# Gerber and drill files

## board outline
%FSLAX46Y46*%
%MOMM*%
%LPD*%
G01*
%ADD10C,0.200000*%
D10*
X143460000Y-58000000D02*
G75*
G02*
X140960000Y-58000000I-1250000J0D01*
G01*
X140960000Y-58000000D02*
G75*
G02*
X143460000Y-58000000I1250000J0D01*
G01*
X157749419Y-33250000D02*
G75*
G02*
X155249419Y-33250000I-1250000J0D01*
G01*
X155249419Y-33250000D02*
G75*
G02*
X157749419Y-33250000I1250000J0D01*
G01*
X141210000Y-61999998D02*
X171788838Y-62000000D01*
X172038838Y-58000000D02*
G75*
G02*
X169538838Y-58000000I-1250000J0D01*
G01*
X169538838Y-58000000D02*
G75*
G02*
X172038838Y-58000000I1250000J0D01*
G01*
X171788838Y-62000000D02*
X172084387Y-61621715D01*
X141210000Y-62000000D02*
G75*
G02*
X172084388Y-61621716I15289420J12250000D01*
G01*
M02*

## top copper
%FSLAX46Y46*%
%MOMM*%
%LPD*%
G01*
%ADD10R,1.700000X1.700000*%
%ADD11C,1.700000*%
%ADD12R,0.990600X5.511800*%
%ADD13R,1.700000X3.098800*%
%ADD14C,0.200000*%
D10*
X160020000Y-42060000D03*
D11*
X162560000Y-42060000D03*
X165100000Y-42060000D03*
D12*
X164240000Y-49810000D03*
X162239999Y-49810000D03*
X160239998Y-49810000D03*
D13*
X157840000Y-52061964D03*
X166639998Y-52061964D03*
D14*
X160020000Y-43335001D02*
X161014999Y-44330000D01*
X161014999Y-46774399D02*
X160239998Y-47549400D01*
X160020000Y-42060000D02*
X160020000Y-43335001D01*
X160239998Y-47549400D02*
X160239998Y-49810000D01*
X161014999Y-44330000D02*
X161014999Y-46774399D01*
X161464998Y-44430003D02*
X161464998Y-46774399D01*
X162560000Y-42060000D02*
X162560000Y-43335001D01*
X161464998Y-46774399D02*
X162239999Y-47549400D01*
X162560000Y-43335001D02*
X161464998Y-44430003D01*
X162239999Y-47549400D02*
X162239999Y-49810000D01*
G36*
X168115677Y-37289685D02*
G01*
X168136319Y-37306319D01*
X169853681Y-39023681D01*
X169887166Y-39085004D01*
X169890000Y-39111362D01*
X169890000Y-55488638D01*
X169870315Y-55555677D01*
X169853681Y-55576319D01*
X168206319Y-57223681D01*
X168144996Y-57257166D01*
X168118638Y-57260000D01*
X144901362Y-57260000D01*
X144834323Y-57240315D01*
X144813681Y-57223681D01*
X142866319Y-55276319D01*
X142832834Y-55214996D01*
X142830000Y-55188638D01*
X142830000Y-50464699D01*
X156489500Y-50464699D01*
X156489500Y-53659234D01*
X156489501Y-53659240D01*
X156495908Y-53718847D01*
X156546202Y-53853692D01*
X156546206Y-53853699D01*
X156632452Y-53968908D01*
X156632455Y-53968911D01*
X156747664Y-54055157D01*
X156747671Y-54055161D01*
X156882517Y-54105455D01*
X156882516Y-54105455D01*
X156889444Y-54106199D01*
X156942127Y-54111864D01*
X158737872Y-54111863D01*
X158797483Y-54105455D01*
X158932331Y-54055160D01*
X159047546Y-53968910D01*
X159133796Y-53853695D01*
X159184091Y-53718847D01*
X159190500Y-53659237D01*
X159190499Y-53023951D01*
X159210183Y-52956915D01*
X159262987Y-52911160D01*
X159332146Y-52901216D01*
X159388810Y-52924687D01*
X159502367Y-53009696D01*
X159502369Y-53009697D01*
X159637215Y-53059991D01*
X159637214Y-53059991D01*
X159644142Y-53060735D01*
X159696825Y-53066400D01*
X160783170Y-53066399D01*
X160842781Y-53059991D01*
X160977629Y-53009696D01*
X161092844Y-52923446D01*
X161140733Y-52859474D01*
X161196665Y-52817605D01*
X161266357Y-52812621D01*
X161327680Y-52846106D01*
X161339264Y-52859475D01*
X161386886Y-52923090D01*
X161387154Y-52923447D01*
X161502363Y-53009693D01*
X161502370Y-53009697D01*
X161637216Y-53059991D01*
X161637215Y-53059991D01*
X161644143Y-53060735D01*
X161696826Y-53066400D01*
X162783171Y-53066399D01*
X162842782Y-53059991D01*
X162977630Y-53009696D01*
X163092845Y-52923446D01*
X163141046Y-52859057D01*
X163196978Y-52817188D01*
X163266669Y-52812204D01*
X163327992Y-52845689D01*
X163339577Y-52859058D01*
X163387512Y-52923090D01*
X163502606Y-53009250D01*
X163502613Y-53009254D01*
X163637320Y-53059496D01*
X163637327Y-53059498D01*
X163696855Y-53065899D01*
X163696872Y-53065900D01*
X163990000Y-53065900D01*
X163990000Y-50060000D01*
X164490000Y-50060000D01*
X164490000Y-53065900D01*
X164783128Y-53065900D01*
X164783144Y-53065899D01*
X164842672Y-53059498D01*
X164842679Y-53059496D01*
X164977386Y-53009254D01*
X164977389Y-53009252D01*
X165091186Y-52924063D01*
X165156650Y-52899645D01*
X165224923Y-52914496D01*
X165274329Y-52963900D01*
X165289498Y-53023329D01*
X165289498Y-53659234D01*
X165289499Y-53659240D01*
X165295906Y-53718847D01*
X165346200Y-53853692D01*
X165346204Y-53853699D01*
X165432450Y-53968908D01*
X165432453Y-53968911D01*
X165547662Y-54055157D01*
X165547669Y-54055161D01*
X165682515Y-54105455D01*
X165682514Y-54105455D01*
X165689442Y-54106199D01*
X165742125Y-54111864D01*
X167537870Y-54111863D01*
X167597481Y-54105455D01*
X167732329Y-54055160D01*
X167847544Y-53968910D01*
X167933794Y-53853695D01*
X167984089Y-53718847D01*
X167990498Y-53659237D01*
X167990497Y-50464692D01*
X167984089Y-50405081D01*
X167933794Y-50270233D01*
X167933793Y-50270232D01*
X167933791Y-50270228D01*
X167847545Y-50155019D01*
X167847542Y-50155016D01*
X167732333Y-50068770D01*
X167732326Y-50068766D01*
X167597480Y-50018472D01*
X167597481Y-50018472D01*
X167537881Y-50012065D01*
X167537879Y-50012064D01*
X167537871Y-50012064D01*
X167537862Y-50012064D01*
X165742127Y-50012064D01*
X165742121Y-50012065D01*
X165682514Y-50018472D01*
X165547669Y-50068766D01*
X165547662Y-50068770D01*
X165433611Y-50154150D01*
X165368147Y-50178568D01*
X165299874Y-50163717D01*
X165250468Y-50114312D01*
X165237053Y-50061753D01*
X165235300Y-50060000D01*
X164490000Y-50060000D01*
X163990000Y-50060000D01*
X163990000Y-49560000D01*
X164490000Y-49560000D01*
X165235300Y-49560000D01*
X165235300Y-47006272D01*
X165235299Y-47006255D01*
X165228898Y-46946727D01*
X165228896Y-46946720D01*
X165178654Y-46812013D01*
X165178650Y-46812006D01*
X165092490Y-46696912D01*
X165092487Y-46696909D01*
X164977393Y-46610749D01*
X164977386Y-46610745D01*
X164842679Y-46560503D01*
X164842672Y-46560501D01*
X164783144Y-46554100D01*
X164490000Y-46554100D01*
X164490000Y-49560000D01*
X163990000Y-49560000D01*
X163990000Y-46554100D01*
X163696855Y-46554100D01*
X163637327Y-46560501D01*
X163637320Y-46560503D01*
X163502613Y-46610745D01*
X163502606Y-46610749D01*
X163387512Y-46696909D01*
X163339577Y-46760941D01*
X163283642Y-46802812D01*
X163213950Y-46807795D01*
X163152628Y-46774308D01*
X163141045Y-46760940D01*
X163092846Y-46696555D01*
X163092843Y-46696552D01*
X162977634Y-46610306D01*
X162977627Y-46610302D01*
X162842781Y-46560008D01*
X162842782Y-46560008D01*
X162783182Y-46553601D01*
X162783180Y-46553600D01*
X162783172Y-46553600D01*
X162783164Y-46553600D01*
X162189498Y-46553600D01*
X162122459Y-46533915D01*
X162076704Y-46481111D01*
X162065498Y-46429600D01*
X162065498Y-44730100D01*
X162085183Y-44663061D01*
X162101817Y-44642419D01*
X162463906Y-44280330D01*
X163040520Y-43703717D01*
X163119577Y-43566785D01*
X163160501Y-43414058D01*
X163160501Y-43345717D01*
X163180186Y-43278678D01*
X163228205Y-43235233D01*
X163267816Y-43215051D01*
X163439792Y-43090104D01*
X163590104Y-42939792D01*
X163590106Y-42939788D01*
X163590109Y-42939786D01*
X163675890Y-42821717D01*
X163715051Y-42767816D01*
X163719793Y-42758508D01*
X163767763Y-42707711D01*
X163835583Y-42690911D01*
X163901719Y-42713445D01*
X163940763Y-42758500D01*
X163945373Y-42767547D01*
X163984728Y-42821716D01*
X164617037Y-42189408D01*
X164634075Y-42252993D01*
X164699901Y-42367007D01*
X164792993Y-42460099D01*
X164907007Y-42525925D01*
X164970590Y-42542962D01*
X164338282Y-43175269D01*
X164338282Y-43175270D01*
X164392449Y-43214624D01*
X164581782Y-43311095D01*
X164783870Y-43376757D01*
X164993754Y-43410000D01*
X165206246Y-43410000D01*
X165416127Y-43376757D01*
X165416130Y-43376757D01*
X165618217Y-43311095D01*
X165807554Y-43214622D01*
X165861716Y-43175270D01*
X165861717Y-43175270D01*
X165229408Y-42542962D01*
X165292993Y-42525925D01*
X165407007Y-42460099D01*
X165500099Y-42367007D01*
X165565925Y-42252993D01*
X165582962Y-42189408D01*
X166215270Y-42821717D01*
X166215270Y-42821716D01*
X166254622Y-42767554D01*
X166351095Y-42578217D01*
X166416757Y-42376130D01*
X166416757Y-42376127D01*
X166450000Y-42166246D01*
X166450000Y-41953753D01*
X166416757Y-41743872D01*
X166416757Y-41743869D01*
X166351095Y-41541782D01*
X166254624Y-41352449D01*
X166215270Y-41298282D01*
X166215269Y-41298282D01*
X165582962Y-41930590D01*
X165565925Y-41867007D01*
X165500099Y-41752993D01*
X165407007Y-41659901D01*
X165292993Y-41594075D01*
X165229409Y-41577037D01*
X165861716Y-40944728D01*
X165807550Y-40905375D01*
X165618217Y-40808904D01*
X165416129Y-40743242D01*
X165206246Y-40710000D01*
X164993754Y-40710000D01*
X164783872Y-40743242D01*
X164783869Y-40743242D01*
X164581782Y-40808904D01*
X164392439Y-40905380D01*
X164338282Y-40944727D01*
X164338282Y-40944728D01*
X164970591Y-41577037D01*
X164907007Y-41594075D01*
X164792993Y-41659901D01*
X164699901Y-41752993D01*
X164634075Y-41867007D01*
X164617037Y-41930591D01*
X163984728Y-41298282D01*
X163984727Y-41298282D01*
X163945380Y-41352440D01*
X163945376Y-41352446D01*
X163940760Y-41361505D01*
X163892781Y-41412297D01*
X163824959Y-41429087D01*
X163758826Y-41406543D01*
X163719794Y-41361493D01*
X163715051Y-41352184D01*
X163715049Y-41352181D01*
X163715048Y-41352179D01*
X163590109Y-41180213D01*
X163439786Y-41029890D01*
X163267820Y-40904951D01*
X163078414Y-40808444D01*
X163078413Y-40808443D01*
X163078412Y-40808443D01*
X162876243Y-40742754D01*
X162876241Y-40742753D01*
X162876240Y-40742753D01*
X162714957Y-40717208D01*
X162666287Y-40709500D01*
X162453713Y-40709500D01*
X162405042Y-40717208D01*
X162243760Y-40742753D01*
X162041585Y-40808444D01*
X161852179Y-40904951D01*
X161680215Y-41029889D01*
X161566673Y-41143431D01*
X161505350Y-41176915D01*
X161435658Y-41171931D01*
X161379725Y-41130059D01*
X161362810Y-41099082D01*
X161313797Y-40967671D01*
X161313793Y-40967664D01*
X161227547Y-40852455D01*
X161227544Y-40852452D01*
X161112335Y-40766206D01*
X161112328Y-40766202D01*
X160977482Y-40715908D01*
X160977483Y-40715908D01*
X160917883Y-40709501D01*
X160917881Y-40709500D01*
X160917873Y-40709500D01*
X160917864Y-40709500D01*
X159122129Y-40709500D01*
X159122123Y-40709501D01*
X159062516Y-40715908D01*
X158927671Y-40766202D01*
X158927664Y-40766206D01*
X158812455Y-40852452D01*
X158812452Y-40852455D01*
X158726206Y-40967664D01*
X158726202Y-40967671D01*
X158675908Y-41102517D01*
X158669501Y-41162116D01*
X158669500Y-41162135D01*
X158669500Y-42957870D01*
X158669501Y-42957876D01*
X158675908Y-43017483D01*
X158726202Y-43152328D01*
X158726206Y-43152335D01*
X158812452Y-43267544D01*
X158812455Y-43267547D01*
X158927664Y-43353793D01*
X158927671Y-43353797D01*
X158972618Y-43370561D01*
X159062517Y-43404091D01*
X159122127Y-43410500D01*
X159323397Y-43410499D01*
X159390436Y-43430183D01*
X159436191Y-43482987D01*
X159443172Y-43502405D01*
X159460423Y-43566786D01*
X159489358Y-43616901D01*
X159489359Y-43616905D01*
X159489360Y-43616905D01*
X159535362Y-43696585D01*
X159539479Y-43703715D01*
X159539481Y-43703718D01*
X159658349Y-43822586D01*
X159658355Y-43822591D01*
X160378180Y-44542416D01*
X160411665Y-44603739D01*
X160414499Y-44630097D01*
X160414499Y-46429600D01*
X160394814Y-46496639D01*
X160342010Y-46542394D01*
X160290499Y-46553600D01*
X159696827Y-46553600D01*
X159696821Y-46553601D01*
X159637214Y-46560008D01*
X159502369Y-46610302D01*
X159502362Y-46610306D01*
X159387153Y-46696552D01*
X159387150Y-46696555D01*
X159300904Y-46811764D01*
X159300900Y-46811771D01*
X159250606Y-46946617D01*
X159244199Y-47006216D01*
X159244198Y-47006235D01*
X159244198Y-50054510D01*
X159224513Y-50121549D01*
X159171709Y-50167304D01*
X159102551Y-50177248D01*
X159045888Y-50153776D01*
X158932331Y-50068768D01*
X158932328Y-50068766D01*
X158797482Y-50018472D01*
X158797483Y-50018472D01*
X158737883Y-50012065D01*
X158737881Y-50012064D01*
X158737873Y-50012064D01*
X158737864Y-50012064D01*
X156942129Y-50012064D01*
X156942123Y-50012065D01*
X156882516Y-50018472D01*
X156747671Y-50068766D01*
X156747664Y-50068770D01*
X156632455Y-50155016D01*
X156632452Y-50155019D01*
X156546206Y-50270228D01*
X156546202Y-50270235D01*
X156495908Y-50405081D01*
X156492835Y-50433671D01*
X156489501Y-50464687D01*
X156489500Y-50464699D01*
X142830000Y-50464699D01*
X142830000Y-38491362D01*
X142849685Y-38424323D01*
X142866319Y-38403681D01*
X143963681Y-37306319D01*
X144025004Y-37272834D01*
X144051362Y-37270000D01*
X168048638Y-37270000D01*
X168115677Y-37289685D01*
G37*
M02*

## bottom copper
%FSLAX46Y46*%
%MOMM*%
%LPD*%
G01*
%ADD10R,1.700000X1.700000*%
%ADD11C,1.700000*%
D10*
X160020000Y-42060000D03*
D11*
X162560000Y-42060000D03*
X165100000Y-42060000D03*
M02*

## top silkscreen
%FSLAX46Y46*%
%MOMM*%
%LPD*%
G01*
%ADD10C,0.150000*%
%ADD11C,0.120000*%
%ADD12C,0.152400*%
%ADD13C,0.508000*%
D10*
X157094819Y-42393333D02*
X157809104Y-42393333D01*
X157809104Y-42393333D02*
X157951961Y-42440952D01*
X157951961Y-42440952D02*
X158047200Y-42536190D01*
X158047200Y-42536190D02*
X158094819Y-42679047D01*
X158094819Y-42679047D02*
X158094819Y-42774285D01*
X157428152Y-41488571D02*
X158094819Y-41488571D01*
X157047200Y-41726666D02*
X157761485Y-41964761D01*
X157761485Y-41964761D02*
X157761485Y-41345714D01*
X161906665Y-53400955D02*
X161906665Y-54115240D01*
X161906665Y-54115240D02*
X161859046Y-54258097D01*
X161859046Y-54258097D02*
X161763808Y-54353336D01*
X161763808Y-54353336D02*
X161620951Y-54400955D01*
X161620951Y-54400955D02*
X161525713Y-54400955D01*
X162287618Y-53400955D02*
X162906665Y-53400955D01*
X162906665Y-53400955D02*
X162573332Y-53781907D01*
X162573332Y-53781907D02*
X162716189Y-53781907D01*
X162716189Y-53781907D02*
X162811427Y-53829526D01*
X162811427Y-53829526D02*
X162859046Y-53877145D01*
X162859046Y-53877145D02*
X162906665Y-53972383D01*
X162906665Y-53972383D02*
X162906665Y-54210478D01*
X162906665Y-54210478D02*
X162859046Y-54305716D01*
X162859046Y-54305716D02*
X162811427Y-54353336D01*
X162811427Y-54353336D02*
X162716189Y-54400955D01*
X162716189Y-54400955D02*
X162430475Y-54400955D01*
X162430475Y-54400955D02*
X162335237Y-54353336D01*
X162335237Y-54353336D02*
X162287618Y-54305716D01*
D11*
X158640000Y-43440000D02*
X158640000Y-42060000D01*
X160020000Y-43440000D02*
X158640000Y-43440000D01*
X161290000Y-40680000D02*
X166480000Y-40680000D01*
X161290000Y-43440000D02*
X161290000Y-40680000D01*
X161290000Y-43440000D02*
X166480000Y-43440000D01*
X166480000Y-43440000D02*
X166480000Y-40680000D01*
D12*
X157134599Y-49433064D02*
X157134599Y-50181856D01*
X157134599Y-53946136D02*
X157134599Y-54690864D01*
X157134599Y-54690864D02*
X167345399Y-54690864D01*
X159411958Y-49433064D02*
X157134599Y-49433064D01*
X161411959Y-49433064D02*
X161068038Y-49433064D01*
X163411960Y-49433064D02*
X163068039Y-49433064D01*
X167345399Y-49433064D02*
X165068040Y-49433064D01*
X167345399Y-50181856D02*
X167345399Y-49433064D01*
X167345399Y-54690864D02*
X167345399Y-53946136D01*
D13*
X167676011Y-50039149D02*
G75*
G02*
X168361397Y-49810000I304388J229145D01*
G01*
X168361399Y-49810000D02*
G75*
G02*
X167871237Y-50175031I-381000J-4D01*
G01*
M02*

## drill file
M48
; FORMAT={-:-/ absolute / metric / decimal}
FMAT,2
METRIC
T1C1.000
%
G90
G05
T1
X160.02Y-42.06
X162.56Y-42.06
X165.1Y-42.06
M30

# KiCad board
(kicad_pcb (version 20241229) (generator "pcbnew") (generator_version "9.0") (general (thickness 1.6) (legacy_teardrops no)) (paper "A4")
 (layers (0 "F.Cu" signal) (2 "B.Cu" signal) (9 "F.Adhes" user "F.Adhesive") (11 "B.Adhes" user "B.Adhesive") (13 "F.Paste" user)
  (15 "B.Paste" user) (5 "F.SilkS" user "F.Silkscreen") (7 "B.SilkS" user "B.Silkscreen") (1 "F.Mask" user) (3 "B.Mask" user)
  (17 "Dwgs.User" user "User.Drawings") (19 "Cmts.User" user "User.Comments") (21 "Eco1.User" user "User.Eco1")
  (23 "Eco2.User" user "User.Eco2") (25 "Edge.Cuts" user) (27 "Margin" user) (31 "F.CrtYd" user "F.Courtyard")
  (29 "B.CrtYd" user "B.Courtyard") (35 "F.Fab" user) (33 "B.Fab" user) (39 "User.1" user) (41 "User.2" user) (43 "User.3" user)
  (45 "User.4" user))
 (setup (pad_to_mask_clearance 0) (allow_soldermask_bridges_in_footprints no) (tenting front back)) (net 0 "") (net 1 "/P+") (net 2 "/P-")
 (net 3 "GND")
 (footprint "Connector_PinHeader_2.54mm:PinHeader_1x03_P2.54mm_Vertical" (layer "F.Cu") (at 160.02 42.06 90)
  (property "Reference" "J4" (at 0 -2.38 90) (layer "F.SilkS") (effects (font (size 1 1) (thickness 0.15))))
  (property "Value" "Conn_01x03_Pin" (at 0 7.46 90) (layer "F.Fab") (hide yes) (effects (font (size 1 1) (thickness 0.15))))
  (fp_line (start -1.38 -1.38) (end 0 -1.38) (stroke (width 0.12) (type solid)) (layer "F.SilkS"))
  (fp_line (start -1.38 0) (end -1.38 -1.38) (stroke (width 0.12) (type solid)) (layer "F.SilkS"))
  (fp_line (start 1.38 1.27) (end 1.38 6.46) (stroke (width 0.12) (type solid)) (layer "F.SilkS"))
  (fp_line (start -1.38 1.27) (end 1.38 1.27) (stroke (width 0.12) (type solid)) (layer "F.SilkS"))
  (fp_line (start -1.38 1.27) (end -1.38 6.46) (stroke (width 0.12) (type solid)) (layer "F.SilkS"))
  (fp_line (start -1.38 6.46) (end 1.38 6.46) (stroke (width 0.12) (type solid)) (layer "F.SilkS"))
  (pad "1" thru_hole rect (at 0 0 90) (size 1.7 1.7) (drill 1) (layers "*.Cu" "*.Mask") (remove_unused_layers no) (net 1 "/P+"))
  (pad "2" thru_hole circle (at 0 2.54 90) (size 1.7 1.7) (drill 1) (layers "*.Cu" "*.Mask") (remove_unused_layers no) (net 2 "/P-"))
  (pad "3" thru_hole circle (at 0 5.08 90) (size 1.7 1.7) (drill 1) (layers "*.Cu" "*.Mask") (remove_unused_layers no) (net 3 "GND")))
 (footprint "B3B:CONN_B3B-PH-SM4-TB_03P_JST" (layer "F.Cu") (at 162.239999 52.061964)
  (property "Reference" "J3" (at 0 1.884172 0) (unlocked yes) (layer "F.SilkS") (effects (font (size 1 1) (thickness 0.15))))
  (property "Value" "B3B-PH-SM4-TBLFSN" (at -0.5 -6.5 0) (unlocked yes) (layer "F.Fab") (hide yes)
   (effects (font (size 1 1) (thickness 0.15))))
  (fp_line (start -5.1054 -2.6289) (end -5.1054 -1.880108) (stroke (width 0.1524) (type solid)) (layer "F.SilkS"))
  (fp_line (start -5.1054 1.884172) (end -5.1054 2.6289) (stroke (width 0.1524) (type solid)) (layer "F.SilkS"))
  (fp_line (start -5.1054 2.6289) (end 5.1054 2.6289) (stroke (width 0.1524) (type solid)) (layer "F.SilkS"))
  (fp_line (start -2.828041 -2.6289) (end -5.1054 -2.6289) (stroke (width 0.1524) (type solid)) (layer "F.SilkS"))
  (fp_line (start -0.82804 -2.6289) (end -1.171961 -2.6289) (stroke (width 0.1524) (type solid)) (layer "F.SilkS"))
  (fp_line (start 1.171961 -2.6289) (end 0.82804 -2.6289) (stroke (width 0.1524) (type solid)) (layer "F.SilkS"))
  (fp_line (start 5.1054 -2.6289) (end 2.828041 -2.6289) (stroke (width 0.1524) (type solid)) (layer "F.SilkS"))
  (fp_line (start 5.1054 -1.880108) (end 5.1054 -2.6289) (stroke (width 0.1524) (type solid)) (layer "F.SilkS"))
  (fp_line (start 5.1054 2.6289) (end 5.1054 1.884172) (stroke (width 0.1524) (type solid)) (layer "F.SilkS"))
  (fp_arc (start 5.436012 -2.022815) (mid 5.619592 -2.613304) (end 6.1214 -2.251964) (stroke (width 0.508) (type solid)) (layer "F.SilkS"))
  (fp_arc (start 6.1214 -2.251964) (mid 5.967964 -1.94639) (end 5.631239 -1.886937) (stroke (width 0.508) (type solid)) (layer "F.SilkS"))
  (pad "1" smd rect (at 2.000001 -2.251964) (size 0.9906 5.5118) (layers "F.Cu" "F.Mask" "F.Paste") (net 3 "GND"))
  (pad "2" smd rect (at 0 -2.251964) (size 0.9906 5.5118) (layers "F.Cu" "F.Mask" "F.Paste") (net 2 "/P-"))
  (pad "3" smd rect (at -2.000001 -2.251964) (size 0.9906 5.5118) (layers "F.Cu" "F.Mask" "F.Paste") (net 1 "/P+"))
  (pad "4" smd rect (at -4.399999 0) (size 1.7 3.0988) (layers "F.Cu" "F.Mask" "F.Paste"))
  (pad "5" smd rect (at 4.399999 0) (size 1.7 3.0988) (layers "F.Cu" "F.Mask" "F.Paste")))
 (gr_circle (center 142.21 58) (end 143.46 58) (stroke (width 0.2) (type solid)) (fill no) (layer "Edge.Cuts"))
 (gr_circle (center 156.499419 33.25) (end 157.749419 33.25) (stroke (width 0.2) (type solid)) (fill no) (layer "Edge.Cuts"))
 (gr_line (start 141.21 61.999998) (end 171.788838 62) (stroke (width 0.2) (type solid)) (layer "Edge.Cuts"))
 (gr_circle (center 170.788838 58) (end 172.038838 58) (stroke (width 0.2) (type solid)) (fill no) (layer "Edge.Cuts"))
 (gr_line (start 171.788838 62) (end 172.084387 61.621715) (stroke (width 0.2) (type solid)) (layer "Edge.Cuts"))
 (gr_arc (start 141.21 62) (mid 156.259394 30.15992) (end 172.084387 61.621715) (stroke (width 0.2) (type solid)) (layer "Edge.Cuts"))
 (segment (start 160.02 43.335001) (end 161.014999 44.33) (width 0.2) (layer "F.Cu") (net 1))
 (segment (start 161.014999 46.774399) (end 160.239998 47.5494) (width 0.2) (layer "F.Cu") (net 1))
 (segment (start 160.02 42.06) (end 160.02 43.335001) (width 0.2) (layer "F.Cu") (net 1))
 (segment (start 160.239998 47.5494) (end 160.239998 49.81) (width 0.2) (layer "F.Cu") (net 1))
 (segment (start 161.014999 44.33) (end 161.014999 46.774399) (width 0.2) (layer "F.Cu") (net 1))
 (segment (start 161.464998 44.430003) (end 161.464998 46.774399) (width 0.2) (layer "F.Cu") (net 2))
 (segment (start 162.56 42.06) (end 162.56 43.335001) (width 0.2) (layer "F.Cu") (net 2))
 (segment (start 161.464998 46.774399) (end 162.239999 47.5494) (width 0.2) (layer "F.Cu") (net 2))
 (segment (start 162.56 43.335001) (end 161.464998 44.430003) (width 0.2) (layer "F.Cu") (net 2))
 (segment (start 162.239999 47.5494) (end 162.239999 49.81) (width 0.2) (layer "F.Cu") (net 2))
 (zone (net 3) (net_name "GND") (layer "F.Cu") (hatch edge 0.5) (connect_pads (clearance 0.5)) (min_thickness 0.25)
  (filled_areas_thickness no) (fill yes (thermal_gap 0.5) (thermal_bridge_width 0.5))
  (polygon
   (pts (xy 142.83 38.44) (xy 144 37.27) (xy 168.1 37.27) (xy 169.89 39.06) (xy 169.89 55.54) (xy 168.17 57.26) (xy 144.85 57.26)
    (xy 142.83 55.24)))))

